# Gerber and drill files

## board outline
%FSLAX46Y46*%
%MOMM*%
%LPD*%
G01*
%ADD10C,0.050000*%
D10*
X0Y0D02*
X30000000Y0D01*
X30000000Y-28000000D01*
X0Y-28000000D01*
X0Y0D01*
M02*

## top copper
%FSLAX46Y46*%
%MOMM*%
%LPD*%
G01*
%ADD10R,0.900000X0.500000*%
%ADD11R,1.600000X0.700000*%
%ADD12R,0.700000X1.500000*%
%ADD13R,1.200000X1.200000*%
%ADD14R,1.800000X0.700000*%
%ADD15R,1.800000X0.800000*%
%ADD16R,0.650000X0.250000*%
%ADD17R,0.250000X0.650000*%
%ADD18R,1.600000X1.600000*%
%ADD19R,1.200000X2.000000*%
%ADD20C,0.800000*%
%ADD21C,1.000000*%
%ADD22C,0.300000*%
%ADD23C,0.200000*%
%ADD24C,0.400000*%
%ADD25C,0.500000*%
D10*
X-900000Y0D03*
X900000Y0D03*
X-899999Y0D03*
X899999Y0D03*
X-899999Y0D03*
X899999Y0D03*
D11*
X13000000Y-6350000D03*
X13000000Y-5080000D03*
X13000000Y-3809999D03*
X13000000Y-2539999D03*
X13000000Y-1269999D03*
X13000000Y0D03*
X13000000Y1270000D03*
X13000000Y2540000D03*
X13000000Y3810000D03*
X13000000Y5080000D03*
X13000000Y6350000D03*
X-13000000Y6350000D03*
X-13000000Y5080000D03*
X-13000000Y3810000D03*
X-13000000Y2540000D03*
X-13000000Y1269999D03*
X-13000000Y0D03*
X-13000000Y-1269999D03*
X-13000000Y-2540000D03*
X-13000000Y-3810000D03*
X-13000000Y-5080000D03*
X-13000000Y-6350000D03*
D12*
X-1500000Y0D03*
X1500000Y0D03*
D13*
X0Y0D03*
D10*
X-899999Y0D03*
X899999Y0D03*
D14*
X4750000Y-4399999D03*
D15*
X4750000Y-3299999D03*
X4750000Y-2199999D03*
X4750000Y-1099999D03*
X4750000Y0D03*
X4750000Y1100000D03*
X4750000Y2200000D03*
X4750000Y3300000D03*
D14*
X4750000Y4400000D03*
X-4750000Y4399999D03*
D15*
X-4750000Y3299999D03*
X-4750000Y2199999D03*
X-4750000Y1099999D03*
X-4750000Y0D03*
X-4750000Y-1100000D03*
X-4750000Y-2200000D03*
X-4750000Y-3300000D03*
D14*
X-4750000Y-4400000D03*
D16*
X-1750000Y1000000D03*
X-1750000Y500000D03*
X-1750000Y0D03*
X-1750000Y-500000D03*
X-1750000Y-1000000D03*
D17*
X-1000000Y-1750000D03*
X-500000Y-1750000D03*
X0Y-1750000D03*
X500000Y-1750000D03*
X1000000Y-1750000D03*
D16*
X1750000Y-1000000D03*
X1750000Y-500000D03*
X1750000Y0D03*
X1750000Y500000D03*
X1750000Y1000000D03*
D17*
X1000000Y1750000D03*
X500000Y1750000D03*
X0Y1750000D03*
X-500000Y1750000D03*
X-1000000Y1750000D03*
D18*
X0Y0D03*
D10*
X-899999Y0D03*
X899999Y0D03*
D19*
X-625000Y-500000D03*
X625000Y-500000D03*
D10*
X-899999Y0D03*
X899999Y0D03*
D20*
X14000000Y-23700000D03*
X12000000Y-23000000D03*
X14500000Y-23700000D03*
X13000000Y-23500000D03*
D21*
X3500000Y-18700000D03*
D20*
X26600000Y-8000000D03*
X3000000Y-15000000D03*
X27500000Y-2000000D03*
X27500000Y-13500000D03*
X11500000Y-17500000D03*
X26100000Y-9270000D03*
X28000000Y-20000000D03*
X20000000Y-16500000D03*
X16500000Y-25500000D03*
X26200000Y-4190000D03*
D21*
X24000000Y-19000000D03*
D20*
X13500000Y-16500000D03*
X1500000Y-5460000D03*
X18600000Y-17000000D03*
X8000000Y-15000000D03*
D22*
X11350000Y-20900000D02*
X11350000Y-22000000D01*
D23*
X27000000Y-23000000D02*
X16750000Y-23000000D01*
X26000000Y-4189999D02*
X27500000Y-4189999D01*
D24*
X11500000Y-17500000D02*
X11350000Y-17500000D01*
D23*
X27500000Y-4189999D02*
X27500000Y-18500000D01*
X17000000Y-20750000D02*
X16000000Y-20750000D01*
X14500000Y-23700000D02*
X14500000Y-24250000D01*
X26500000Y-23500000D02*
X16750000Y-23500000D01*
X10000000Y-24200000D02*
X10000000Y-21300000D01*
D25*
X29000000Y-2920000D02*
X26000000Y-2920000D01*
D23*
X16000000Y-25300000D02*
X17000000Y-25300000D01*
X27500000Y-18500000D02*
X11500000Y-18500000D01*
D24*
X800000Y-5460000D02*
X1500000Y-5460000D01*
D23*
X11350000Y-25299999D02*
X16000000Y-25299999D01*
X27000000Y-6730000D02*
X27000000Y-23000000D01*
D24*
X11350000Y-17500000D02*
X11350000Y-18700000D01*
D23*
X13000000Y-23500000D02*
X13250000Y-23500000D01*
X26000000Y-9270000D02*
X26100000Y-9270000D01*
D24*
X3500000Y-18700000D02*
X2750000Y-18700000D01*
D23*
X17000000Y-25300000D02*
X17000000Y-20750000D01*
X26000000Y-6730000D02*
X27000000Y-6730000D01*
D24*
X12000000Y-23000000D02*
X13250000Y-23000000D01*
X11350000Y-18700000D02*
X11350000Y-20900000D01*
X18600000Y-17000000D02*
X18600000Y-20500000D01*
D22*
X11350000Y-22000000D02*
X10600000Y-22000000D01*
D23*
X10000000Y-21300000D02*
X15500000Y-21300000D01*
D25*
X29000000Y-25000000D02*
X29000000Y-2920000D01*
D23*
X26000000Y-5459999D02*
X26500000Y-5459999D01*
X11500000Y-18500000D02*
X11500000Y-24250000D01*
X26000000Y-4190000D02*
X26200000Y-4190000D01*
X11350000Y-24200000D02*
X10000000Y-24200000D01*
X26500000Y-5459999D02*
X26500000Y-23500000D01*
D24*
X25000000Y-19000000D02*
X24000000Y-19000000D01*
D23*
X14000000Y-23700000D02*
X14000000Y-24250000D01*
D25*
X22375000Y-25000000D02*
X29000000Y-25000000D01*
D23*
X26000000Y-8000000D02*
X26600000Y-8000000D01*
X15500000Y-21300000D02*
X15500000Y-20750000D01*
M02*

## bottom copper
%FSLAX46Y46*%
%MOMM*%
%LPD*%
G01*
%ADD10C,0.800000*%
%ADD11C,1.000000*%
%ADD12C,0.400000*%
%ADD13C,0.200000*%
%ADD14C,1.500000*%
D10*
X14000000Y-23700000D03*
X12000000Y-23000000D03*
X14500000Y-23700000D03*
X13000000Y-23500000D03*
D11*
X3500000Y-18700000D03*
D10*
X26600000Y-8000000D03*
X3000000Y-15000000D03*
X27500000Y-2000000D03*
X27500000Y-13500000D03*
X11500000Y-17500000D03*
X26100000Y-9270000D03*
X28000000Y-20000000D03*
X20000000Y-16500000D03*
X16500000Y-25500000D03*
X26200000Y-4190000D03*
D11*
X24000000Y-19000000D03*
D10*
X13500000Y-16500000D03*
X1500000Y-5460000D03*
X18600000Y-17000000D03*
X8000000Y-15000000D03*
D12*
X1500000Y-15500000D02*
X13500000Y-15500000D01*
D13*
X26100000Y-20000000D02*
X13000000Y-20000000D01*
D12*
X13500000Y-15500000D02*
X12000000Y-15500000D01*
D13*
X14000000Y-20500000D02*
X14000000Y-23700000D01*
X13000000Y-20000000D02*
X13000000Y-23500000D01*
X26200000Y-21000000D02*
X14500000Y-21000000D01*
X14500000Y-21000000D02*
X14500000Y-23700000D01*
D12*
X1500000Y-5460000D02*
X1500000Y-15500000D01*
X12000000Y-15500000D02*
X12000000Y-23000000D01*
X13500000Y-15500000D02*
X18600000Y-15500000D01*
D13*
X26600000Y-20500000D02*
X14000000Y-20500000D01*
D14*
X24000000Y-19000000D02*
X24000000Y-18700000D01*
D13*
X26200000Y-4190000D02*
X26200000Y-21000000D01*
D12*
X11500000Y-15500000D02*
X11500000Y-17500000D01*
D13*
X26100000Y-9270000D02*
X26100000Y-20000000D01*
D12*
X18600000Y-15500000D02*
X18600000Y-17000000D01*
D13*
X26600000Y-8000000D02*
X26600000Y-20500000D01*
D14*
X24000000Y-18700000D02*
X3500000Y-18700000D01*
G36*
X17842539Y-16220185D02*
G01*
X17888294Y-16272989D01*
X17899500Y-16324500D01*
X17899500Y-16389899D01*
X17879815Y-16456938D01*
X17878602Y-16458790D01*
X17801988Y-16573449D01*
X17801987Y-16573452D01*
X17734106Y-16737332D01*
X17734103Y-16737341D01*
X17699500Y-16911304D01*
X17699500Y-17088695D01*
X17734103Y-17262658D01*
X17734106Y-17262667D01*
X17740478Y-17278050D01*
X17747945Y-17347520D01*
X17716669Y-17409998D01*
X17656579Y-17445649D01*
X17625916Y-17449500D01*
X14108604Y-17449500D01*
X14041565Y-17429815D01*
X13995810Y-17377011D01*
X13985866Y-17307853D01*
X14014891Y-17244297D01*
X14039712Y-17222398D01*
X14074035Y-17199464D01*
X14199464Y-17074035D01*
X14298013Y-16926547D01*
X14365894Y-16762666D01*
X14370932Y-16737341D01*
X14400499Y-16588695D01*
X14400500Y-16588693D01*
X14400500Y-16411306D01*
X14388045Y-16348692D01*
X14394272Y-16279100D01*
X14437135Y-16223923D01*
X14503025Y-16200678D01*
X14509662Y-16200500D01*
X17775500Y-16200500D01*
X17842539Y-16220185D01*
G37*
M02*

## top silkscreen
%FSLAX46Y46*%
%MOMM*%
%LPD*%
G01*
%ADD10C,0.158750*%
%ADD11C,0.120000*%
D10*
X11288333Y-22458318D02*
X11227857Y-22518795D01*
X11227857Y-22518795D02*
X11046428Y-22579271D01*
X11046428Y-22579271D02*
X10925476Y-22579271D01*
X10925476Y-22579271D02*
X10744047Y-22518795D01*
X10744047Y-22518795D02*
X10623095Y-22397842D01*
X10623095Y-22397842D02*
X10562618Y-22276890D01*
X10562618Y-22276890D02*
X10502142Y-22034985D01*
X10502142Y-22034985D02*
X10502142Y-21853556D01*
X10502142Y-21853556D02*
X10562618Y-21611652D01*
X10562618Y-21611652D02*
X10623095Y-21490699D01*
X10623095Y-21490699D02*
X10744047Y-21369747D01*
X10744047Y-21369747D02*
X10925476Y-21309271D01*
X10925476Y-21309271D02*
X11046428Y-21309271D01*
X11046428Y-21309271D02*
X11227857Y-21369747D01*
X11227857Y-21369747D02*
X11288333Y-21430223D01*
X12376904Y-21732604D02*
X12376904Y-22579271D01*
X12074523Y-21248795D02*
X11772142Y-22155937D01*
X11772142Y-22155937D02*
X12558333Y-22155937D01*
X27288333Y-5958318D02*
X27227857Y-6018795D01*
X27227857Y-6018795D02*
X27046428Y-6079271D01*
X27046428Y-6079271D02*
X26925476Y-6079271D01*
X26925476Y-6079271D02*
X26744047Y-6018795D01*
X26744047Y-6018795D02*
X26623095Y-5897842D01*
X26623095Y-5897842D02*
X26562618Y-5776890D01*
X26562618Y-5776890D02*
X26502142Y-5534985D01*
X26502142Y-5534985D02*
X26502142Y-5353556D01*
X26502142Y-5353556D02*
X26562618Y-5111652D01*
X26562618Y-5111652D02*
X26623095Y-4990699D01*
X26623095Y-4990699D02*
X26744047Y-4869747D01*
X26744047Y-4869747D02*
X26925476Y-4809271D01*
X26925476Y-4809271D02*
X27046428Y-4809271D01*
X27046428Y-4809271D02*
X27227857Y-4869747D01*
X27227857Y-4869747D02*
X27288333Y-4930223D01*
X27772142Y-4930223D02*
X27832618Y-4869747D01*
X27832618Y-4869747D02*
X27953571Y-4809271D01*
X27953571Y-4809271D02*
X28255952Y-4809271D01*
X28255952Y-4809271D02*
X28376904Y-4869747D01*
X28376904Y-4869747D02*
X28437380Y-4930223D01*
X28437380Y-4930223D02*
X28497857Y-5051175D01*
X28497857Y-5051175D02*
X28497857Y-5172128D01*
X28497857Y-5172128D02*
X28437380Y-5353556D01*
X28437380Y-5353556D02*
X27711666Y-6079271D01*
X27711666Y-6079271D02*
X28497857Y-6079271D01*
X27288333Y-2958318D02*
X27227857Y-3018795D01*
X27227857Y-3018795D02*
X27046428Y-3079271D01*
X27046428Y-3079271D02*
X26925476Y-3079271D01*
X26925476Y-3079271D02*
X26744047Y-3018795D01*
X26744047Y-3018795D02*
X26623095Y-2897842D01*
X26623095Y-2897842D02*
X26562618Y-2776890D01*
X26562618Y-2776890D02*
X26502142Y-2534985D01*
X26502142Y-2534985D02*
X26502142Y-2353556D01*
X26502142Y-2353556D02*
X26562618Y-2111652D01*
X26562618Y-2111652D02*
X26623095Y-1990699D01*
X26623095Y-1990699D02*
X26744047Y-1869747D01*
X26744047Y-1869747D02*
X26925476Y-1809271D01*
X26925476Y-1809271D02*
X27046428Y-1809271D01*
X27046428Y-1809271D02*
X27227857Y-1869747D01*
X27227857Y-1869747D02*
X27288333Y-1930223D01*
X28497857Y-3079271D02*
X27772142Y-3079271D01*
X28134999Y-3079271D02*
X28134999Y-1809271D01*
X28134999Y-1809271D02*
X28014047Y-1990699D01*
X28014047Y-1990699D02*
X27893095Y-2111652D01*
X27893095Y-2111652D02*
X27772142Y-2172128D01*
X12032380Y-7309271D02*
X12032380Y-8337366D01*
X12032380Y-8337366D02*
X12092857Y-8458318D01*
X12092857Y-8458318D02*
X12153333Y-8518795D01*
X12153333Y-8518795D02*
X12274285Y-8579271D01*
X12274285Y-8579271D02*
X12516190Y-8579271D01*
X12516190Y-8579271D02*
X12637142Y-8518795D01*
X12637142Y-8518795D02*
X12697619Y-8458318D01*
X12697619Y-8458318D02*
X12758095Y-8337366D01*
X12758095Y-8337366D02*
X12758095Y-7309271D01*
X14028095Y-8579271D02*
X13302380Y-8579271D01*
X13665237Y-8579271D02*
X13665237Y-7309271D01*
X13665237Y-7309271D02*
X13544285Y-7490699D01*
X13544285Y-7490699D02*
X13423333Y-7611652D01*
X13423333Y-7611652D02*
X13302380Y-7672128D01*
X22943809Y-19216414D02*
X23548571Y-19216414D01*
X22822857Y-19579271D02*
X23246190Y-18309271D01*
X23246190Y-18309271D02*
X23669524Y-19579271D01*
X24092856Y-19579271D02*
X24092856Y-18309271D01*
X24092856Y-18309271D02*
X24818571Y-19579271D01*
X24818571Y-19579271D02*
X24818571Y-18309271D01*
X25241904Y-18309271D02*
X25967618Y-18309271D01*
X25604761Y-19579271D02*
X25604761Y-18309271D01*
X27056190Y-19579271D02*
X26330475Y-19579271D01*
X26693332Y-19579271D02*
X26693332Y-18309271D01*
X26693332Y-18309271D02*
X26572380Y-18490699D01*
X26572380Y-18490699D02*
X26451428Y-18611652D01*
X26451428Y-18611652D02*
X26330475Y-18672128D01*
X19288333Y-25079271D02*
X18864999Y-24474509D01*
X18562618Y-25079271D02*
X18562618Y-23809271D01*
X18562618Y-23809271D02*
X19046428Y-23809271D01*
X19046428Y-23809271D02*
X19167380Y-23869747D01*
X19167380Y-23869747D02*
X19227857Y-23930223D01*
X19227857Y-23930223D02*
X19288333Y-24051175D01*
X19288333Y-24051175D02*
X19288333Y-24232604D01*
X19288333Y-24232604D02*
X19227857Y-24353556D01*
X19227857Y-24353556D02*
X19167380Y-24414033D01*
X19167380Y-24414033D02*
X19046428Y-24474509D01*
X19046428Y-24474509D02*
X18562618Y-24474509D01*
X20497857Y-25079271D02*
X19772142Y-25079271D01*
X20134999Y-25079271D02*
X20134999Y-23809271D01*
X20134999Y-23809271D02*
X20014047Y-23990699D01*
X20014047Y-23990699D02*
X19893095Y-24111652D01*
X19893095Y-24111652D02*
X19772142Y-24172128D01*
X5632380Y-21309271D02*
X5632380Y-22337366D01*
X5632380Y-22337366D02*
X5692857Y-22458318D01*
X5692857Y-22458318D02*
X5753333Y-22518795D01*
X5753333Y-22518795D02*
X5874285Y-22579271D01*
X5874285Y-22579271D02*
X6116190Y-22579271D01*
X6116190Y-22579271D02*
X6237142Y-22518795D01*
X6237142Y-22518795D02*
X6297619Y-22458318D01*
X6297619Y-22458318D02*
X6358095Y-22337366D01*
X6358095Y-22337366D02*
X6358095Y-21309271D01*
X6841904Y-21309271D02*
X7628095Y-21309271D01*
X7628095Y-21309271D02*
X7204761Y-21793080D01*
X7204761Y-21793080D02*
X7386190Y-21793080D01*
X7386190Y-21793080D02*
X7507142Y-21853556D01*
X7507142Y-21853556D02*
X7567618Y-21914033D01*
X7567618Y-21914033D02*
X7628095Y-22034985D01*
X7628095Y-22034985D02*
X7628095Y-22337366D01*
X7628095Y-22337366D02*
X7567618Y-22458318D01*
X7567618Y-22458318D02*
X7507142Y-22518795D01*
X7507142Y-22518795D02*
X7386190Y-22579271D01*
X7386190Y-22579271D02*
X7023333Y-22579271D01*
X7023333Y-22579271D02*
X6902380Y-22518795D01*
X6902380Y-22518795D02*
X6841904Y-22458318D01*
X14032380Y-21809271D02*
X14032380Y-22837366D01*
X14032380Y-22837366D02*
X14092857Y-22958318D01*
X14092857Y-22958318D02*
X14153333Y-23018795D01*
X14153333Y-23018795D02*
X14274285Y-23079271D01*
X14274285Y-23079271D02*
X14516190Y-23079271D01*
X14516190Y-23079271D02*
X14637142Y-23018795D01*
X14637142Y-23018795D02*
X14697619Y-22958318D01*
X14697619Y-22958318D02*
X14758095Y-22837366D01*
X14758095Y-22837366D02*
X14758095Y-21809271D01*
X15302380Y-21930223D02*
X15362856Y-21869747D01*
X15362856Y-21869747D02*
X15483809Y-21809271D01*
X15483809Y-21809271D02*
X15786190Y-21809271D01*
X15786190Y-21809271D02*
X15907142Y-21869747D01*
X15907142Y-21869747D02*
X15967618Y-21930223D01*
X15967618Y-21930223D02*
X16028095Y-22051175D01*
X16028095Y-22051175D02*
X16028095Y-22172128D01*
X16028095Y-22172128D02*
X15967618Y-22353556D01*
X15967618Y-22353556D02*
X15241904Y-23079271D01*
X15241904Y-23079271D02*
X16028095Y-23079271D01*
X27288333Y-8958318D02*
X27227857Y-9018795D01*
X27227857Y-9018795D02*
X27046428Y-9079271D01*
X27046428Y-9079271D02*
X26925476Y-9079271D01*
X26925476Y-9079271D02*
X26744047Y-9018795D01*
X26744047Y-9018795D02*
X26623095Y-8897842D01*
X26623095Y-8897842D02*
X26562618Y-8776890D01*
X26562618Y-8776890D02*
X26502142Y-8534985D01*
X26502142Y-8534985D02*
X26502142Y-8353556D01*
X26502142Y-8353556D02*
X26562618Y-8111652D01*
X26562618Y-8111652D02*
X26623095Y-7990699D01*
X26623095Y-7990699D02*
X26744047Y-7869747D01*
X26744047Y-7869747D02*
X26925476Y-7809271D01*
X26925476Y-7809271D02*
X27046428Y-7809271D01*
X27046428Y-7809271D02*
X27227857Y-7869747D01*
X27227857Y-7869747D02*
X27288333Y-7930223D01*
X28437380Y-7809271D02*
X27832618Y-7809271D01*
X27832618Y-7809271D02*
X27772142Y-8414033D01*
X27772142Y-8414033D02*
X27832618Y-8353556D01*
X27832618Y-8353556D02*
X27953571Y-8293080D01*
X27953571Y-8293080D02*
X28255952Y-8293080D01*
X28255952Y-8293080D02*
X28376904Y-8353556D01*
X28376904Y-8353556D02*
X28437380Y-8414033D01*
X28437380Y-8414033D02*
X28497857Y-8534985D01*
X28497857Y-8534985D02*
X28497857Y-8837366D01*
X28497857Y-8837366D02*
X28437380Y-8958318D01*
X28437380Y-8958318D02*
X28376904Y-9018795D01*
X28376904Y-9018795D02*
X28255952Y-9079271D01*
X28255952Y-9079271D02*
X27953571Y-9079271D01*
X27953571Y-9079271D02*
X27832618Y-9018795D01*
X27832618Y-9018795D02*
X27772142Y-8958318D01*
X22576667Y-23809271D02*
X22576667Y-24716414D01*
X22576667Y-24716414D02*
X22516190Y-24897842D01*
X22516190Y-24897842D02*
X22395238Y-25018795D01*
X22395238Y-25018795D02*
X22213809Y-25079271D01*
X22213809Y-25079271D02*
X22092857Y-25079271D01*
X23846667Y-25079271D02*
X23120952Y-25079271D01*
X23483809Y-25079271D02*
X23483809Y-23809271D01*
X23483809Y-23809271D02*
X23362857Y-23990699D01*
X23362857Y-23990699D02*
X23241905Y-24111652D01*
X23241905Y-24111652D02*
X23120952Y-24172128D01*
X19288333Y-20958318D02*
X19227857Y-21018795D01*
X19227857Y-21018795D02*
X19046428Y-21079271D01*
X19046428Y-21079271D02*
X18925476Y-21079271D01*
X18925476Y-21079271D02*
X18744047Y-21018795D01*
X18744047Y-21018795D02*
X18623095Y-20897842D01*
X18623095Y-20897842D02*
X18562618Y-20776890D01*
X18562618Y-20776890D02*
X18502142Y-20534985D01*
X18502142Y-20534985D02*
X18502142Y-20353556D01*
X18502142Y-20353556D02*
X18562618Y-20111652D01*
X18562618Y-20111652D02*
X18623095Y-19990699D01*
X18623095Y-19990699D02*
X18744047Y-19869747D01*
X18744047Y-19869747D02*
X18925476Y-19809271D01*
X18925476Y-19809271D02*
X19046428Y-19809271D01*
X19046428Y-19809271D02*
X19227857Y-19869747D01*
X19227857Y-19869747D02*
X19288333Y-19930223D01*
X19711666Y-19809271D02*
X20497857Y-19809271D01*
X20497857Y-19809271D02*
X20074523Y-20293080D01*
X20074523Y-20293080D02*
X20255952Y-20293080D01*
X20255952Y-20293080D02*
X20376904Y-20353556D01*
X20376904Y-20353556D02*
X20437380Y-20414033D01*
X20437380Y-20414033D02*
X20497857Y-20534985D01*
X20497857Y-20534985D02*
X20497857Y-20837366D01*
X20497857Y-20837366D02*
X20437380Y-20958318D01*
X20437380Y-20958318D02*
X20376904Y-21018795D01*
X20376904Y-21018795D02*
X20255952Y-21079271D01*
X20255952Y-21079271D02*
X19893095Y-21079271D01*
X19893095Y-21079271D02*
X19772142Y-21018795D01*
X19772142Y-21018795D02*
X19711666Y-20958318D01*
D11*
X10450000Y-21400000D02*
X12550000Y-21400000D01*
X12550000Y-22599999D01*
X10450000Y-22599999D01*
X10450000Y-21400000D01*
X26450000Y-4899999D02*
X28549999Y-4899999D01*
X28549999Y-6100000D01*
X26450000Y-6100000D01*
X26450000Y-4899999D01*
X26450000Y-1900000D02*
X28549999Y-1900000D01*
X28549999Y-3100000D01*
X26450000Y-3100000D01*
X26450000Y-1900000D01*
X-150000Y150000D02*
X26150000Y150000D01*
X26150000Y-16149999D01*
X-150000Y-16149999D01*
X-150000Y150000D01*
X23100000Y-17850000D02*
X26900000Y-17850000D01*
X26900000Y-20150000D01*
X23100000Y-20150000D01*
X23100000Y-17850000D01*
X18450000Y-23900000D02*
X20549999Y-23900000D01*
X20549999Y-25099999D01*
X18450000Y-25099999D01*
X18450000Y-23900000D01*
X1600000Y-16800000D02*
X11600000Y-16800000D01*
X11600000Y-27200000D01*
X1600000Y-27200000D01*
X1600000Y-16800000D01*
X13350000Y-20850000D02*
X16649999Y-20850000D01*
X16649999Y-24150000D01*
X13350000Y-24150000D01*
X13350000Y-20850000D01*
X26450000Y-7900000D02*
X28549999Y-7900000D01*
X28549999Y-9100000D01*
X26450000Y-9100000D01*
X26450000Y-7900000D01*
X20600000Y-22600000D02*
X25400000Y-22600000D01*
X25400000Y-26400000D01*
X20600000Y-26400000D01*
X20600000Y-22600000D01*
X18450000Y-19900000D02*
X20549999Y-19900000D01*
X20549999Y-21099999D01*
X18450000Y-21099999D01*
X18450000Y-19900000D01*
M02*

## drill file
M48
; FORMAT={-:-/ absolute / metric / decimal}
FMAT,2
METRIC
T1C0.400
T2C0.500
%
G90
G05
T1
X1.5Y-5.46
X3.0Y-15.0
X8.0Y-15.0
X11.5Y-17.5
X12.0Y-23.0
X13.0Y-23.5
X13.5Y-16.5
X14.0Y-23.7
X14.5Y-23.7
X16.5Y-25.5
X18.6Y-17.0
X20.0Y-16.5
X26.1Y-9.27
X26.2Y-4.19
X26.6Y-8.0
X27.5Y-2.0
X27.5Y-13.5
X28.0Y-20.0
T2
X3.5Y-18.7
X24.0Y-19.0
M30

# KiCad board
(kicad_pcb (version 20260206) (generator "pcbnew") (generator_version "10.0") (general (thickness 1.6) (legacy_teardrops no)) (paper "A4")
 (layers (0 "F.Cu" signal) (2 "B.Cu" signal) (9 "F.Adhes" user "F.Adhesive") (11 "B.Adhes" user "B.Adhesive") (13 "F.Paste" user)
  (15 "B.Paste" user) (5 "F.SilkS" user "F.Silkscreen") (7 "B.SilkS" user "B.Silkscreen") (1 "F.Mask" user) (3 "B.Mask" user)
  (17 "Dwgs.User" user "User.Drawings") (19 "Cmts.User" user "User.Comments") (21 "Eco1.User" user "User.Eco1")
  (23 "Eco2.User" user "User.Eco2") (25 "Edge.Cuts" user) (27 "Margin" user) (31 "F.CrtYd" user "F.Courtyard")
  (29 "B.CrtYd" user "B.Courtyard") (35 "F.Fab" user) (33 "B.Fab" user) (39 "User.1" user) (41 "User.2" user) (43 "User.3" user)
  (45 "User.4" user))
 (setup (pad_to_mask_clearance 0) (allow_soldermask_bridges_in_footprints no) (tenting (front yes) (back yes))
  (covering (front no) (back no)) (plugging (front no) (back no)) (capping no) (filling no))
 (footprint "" (layer "F.Cu") (at 11.5 22)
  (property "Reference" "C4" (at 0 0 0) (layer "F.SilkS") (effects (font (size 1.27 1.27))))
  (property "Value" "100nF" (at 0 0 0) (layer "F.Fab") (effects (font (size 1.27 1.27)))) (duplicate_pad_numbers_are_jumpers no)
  (fp_rect (start -1.05 -0.6) (end 1.05 0.599999) (stroke (width 0.12) (type default)) (fill no) (layer "F.SilkS"))
  (pad "1" smd rect (at -12.4 -22) (size 0.9 0.5) (layers "F.Cu" "F.Mask" "F.Paste") (thermal_bridge_angle 45))
  (pad "2" smd rect (at -10.6 -22) (size 0.9 0.5) (layers "F.Cu" "F.Mask" "F.Paste") (thermal_bridge_angle 45)))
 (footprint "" (layer "F.Cu") (at 27.5 5.5)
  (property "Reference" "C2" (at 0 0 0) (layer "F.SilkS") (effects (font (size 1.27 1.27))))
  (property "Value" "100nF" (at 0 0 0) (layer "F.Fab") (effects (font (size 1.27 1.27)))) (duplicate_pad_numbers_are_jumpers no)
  (fp_rect (start -1.05 -0.600001) (end 1.049999 0.6) (stroke (width 0.12) (type default)) (fill no) (layer "F.SilkS"))
  (pad "1" smd rect (at -28.399999 -5.5) (size 0.9 0.5) (layers "F.Cu" "F.Mask" "F.Paste") (thermal_bridge_angle 45))
  (pad "2" smd rect (at -26.600001 -5.5) (size 0.9 0.5) (layers "F.Cu" "F.Mask" "F.Paste") (thermal_bridge_angle 45)))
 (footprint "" (layer "F.Cu") (at 27.5 2.5)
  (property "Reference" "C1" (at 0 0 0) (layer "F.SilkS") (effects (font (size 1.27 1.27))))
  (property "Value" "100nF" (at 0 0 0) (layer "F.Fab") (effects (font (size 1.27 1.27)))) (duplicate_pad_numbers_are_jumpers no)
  (fp_rect (start -1.05 -0.6) (end 1.049999 0.6) (stroke (width 0.12) (type default)) (fill no) (layer "F.SilkS"))
  (pad "1" smd rect (at -28.399999 -2.5) (size 0.9 0.5) (layers "F.Cu" "F.Mask" "F.Paste") (thermal_bridge_angle 45))
  (pad "2" smd rect (at -26.600001 -2.5) (size 0.9 0.5) (layers "F.Cu" "F.Mask" "F.Paste") (thermal_bridge_angle 45)))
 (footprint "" (layer "F.Cu") (at 13 8)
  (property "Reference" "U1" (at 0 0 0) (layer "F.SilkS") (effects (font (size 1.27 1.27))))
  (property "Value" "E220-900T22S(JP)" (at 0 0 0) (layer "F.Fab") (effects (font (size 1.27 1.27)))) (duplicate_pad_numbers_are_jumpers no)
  (fp_rect (start -13.15 -8.15) (end 13.15 8.149999) (stroke (width 0.12) (type default)) (fill no) (layer "F.SilkS"))
  (pad "1" smd rect (at 0 -1.65) (size 1.6 0.7) (layers "F.Cu" "F.Mask" "F.Paste") (thermal_bridge_angle 45))
  (pad "2" smd rect (at 0 -2.92) (size 1.6 0.7) (layers "F.Cu" "F.Mask" "F.Paste") (thermal_bridge_angle 45))
  (pad "3" smd rect (at 0 -4.190001) (size 1.6 0.7) (layers "F.Cu" "F.Mask" "F.Paste") (thermal_bridge_angle 45))
  (pad "4" smd rect (at 0 -5.460001) (size 1.6 0.7) (layers "F.Cu" "F.Mask" "F.Paste") (thermal_bridge_angle 45))
  (pad "5" smd rect (at 0 -6.730001) (size 1.6 0.7) (layers "F.Cu" "F.Mask" "F.Paste") (thermal_bridge_angle 45))
  (pad "6" smd rect (at 0 -8) (size 1.6 0.7) (layers "F.Cu" "F.Mask" "F.Paste") (thermal_bridge_angle 45))
  (pad "7" smd rect (at 0 -9.27) (size 1.6 0.7) (layers "F.Cu" "F.Mask" "F.Paste") (thermal_bridge_angle 45))
  (pad "8" smd rect (at 0 -10.54) (size 1.6 0.7) (layers "F.Cu" "F.Mask" "F.Paste") (thermal_bridge_angle 45))
  (pad "9" smd rect (at 0 -11.81) (size 1.6 0.7) (layers "F.Cu" "F.Mask" "F.Paste") (thermal_bridge_angle 45))
  (pad "10" smd rect (at 0 -13.08) (size 1.6 0.7) (layers "F.Cu" "F.Mask" "F.Paste") (thermal_bridge_angle 45))
  (pad "11" smd rect (at 0 -14.35) (size 1.6 0.7) (layers "F.Cu" "F.Mask" "F.Paste") (thermal_bridge_angle 45))
  (pad "12" smd rect (at -26 -14.35) (size 1.6 0.7) (layers "F.Cu" "F.Mask" "F.Paste") (thermal_bridge_angle 45))
  (pad "13" smd rect (at -26 -13.08) (size 1.6 0.7) (layers "F.Cu" "F.Mask" "F.Paste") (thermal_bridge_angle 45))
  (pad "14" smd rect (at -26 -11.81) (size 1.6 0.7) (layers "F.Cu" "F.Mask" "F.Paste") (thermal_bridge_angle 45))
  (pad "15" smd rect (at -26 -10.54) (size 1.6 0.7) (layers "F.Cu" "F.Mask" "F.Paste") (thermal_bridge_angle 45))
  (pad "16" smd rect (at -26 -9.269999) (size 1.6 0.7) (layers "F.Cu" "F.Mask" "F.Paste") (thermal_bridge_angle 45))
  (pad "17" smd rect (at -26 -8) (size 1.6 0.7) (layers "F.Cu" "F.Mask" "F.Paste") (thermal_bridge_angle 45))
  (pad "18" smd rect (at -26 -6.730001) (size 1.6 0.7) (layers "F.Cu" "F.Mask" "F.Paste") (thermal_bridge_angle 45))
  (pad "19" smd rect (at -26 -5.46) (size 1.6 0.7) (layers "F.Cu" "F.Mask" "F.Paste") (thermal_bridge_angle 45))
  (pad "20" smd rect (at -26 -4.19) (size 1.6 0.7) (layers "F.Cu" "F.Mask" "F.Paste") (thermal_bridge_angle 45))
  (pad "21" smd rect (at -26 -2.92) (size 1.6 0.7) (layers "F.Cu" "F.Mask" "F.Paste") (thermal_bridge_angle 45))
  (pad "22" smd rect (at -26 -1.65) (size 1.6 0.7) (layers "F.Cu" "F.Mask" "F.Paste") (thermal_bridge_angle 45)))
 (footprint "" (layer "F.Cu") (at 25 19)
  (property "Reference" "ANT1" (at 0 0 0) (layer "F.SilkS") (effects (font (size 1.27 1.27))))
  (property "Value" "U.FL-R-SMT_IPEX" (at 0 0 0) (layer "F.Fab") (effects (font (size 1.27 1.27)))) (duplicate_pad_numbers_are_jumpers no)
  (fp_rect (start -1.9 -1.15) (end 1.9 1.15) (stroke (width 0.12) (type default)) (fill no) (layer "F.SilkS"))
  (pad "G1" smd rect (at -26.5 -19) (size 0.7 1.5) (layers "F.Cu" "F.Mask" "F.Paste") (thermal_bridge_angle 45))
  (pad "G2" smd rect (at -23.5 -19) (size 0.7 1.5) (layers "F.Cu" "F.Mask" "F.Paste") (thermal_bridge_angle 45))
  (pad "S" smd rect (at -25 -19) (size 1.2 1.2) (layers "F.Cu" "F.Mask" "F.Paste") (thermal_bridge_angle 45)))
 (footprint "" (layer "F.Cu") (at 19.5 24.5)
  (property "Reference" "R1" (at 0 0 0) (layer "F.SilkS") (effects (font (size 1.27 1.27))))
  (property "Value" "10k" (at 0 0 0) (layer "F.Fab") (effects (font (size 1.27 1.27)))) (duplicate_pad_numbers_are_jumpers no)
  (fp_rect (start -1.05 -0.6) (end 1.049999 0.599999) (stroke (width 0.12) (type default)) (fill no) (layer "F.SilkS"))
  (pad "1" smd rect (at -20.399999 -24.5) (size 0.9 0.5) (layers "F.Cu" "F.Mask" "F.Paste") (thermal_bridge_angle 45))
  (pad "2" smd rect (at -18.600001 -24.5) (size 0.9 0.5) (layers "F.Cu" "F.Mask" "F.Paste") (thermal_bridge_angle 45)))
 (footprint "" (layer "F.Cu") (at 6.6 22)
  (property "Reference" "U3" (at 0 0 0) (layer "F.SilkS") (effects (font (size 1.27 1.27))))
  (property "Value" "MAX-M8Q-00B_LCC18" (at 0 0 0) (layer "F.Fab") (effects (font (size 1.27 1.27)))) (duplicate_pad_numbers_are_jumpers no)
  (fp_rect (start -5 -5.2) (end 5 5.2) (stroke (width 0.12) (type default)) (fill no) (layer "F.SilkS"))
  (pad "1" smd rect (at -1.85 -17.600001) (size 1.8 0.7) (layers "F.Cu" "F.Mask" "F.Paste") (thermal_bridge_angle 45))
  (pad "2" smd rect (at -1.85 -18.700001) (size 1.8 0.8) (layers "F.Cu" "F.Mask" "F.Paste") (thermal_bridge_angle 45))
  (pad "3" smd rect (at -1.85 -19.800001) (size 1.8 0.8) (layers "F.Cu" "F.Mask" "F.Paste") (thermal_bridge_angle 45))
  (pad "4" smd rect (at -1.85 -20.900001) (size 1.8 0.8) (layers "F.Cu" "F.Mask" "F.Paste") (thermal_bridge_angle 45))
  (pad "5" smd rect (at -1.85 -22) (size 1.8 0.8) (layers "F.Cu" "F.Mask" "F.Paste") (thermal_bridge_angle 45))
  (pad "6" smd rect (at -1.85 -23.1) (size 1.8 0.8) (layers "F.Cu" "F.Mask" "F.Paste") (thermal_bridge_angle 45))
  (pad "7" smd rect (at -1.85 -24.2) (size 1.8 0.8) (layers "F.Cu" "F.Mask" "F.Paste") (thermal_bridge_angle 45))
  (pad "8" smd rect (at -1.85 -25.3) (size 1.8 0.8) (layers "F.Cu" "F.Mask" "F.Paste") (thermal_bridge_angle 45))
  (pad "9" smd rect (at -1.85 -26.4) (size 1.8 0.7) (layers "F.Cu" "F.Mask" "F.Paste") (thermal_bridge_angle 45))
  (pad "10" smd rect (at -11.35 -26.399999) (size 1.8 0.7) (layers "F.Cu" "F.Mask" "F.Paste") (thermal_bridge_angle 45))
  (pad "11" smd rect (at -11.35 -25.299999) (size 1.8 0.8) (layers "F.Cu" "F.Mask" "F.Paste") (thermal_bridge_angle 45))
  (pad "12" smd rect (at -11.35 -24.199999) (size 1.8 0.8) (layers "F.Cu" "F.Mask" "F.Paste") (thermal_bridge_angle 45))
  (pad "13" smd rect (at -11.35 -23.099999) (size 1.8 0.8) (layers "F.Cu" "F.Mask" "F.Paste") (thermal_bridge_angle 45))
  (pad "14" smd rect (at -11.35 -22) (size 1.8 0.8) (layers "F.Cu" "F.Mask" "F.Paste") (thermal_bridge_angle 45))
  (pad "15" smd rect (at -11.35 -20.9) (size 1.8 0.8) (layers "F.Cu" "F.Mask" "F.Paste") (thermal_bridge_angle 45))
  (pad "16" smd rect (at -11.35 -19.8) (size 1.8 0.8) (layers "F.Cu" "F.Mask" "F.Paste") (thermal_bridge_angle 45))
  (pad "17" smd rect (at -11.35 -18.7) (size 1.8 0.8) (layers "F.Cu" "F.Mask" "F.Paste") (thermal_bridge_angle 45))
  (pad "18" smd rect (at -11.35 -17.6) (size 1.8 0.7) (layers "F.Cu" "F.Mask" "F.Paste") (thermal_bridge_angle 45)))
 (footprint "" (layer "F.Cu") (at 15 22.5)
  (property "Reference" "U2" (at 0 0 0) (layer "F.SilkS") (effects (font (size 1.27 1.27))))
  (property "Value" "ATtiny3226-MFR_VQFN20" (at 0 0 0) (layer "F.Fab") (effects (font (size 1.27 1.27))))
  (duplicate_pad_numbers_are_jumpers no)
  (fp_rect (start -1.65 -1.65) (end 1.649999 1.65) (stroke (width 0.12) (type default)) (fill no) (layer "F.SilkS"))
  (pad "1" smd rect (at -16.75 -23.5) (size 0.65 0.25) (layers "F.Cu" "F.Mask" "F.Paste") (thermal_bridge_angle 45))
  (pad "2" smd rect (at -16.75 -23) (size 0.65 0.25) (layers "F.Cu" "F.Mask" "F.Paste") (thermal_bridge_angle 45))
  (pad "3" smd rect (at -16.75 -22.5) (size 0.65 0.25) (layers "F.Cu" "F.Mask" "F.Paste") (thermal_bridge_angle 45))
  (pad "4" smd rect (at -16.75 -22) (size 0.65 0.25) (layers "F.Cu" "F.Mask" "F.Paste") (thermal_bridge_angle 45))
  (pad "5" smd rect (at -16.75 -21.5) (size 0.65 0.25) (layers "F.Cu" "F.Mask" "F.Paste") (thermal_bridge_angle 45))
  (pad "6" smd rect (at -16 -20.75) (size 0.25 0.65) (layers "F.Cu" "F.Mask" "F.Paste") (thermal_bridge_angle 45))
  (pad "7" smd rect (at -15.5 -20.75) (size 0.25 0.65) (layers "F.Cu" "F.Mask" "F.Paste") (thermal_bridge_angle 45))
  (pad "8" smd rect (at -15 -20.75) (size 0.25 0.65) (layers "F.Cu" "F.Mask" "F.Paste") (thermal_bridge_angle 45))
  (pad "9" smd rect (at -14.5 -20.75) (size 0.25 0.65) (layers "F.Cu" "F.Mask" "F.Paste") (thermal_bridge_angle 45))
  (pad "10" smd rect (at -14 -20.75) (size 0.25 0.65) (layers "F.Cu" "F.Mask" "F.Paste") (thermal_bridge_angle 45))
  (pad "11" smd rect (at -13.25 -21.5) (size 0.65 0.25) (layers "F.Cu" "F.Mask" "F.Paste") (thermal_bridge_angle 45))
  (pad "12" smd rect (at -13.25 -22) (size 0.65 0.25) (layers "F.Cu" "F.Mask" "F.Paste") (thermal_bridge_angle 45))
  (pad "13" smd rect (at -13.25 -22.5) (size 0.65 0.25) (layers "F.Cu" "F.Mask" "F.Paste") (thermal_bridge_angle 45))
  (pad "14" smd rect (at -13.25 -23) (size 0.65 0.25) (layers "F.Cu" "F.Mask" "F.Paste") (thermal_bridge_angle 45))
  (pad "15" smd rect (at -13.25 -23.5) (size 0.65 0.25) (layers "F.Cu" "F.Mask" "F.Paste") (thermal_bridge_angle 45))
  (pad "16" smd rect (at -14 -24.25) (size 0.25 0.65) (layers "F.Cu" "F.Mask" "F.Paste") (thermal_bridge_angle 45))
  (pad "17" smd rect (at -14.5 -24.25) (size 0.25 0.65) (layers "F.Cu" "F.Mask" "F.Paste") (thermal_bridge_angle 45))
  (pad "18" smd rect (at -15 -24.25) (size 0.25 0.65) (layers "F.Cu" "F.Mask" "F.Paste") (thermal_bridge_angle 45))
  (pad "19" smd rect (at -15.5 -24.25) (size 0.25 0.65) (layers "F.Cu" "F.Mask" "F.Paste") (thermal_bridge_angle 45))
  (pad "20" smd rect (at -16 -24.25) (size 0.25 0.65) (layers "F.Cu" "F.Mask" "F.Paste") (thermal_bridge_angle 45))
  (pad "EP" smd rect (at -15 -22.5) (size 1.6 1.6) (layers "F.Cu" "F.Mask" "F.Paste") (thermal_bridge_angle 45)))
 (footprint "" (layer "F.Cu") (at 27.5 8.5)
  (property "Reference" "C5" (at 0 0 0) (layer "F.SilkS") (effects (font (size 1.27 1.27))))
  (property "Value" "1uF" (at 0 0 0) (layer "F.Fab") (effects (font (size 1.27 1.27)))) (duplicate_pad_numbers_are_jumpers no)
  (fp_rect (start -1.05 -0.6) (end 1.049999 0.6) (stroke (width 0.12) (type default)) (fill no) (layer "F.SilkS"))
  (pad "1" smd rect (at -28.399999 -8.5) (size 0.9 0.5) (layers "F.Cu" "F.Mask" "F.Paste") (thermal_bridge_angle 45))
  (pad "2" smd rect (at -26.600001 -8.5) (size 0.9 0.5) (layers "F.Cu" "F.Mask" "F.Paste") (thermal_bridge_angle 45)))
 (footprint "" (layer "F.Cu") (at 23 24.5)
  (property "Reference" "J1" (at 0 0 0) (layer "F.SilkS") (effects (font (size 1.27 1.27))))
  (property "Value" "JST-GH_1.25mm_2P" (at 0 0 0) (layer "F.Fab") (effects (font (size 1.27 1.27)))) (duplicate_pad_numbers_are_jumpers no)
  (fp_rect (start -2.4 -1.9) (end 2.4 1.9) (stroke (width 0.12) (type default)) (fill no) (layer "F.SilkS"))
  (pad "1" smd rect (at -23.625 -24) (size 1.2 2) (layers "F.Cu" "F.Mask" "F.Paste") (thermal_bridge_angle 45))
  (pad "2" smd rect (at -22.375 -24) (size 1.2 2) (layers "F.Cu" "F.Mask" "F.Paste") (thermal_bridge_angle 45)))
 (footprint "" (layer "F.Cu") (at 19.5 20.5)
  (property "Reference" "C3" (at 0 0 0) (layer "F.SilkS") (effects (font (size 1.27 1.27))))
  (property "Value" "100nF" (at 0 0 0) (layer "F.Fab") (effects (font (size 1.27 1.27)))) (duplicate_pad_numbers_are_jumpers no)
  (fp_rect (start -1.05 -0.6) (end 1.049999 0.599999) (stroke (width 0.12) (type default)) (fill no) (layer "F.SilkS"))
  (pad "1" smd rect (at -20.399999 -20.5) (size 0.9 0.5) (layers "F.Cu" "F.Mask" "F.Paste") (thermal_bridge_angle 45))
  (pad "2" smd rect (at -18.600001 -20.5) (size 0.9 0.5) (layers "F.Cu" "F.Mask" "F.Paste") (thermal_bridge_angle 45)))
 (gr_rect (start 0 0) (end 30 28) (stroke (width 0.05) (type default)) (fill no) (layer "Edge.Cuts"))
 (segment (start 11.35 20.9) (end 11.35 22) (width 0.3) (layer "F.Cu") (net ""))
 (segment (start 27 23) (end 16.75 23) (width 0.2) (layer "F.Cu") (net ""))
 (segment (start 26 4.189999) (end 27.5 4.189999) (width 0.2) (layer "F.Cu") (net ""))
 (segment (start 11.5 17.5) (end 11.35 17.5) (width 0.4) (layer "F.Cu") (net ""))
 (segment (start 27.5 4.189999) (end 27.5 18.5) (width 0.2) (layer "F.Cu") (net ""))
 (segment (start 17 20.75) (end 16 20.75) (width 0.2) (layer "F.Cu") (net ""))
 (segment (start 14.5 23.7) (end 14.5 24.25) (width 0.2) (layer "F.Cu") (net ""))
 (segment (start 26.5 23.5) (end 16.75 23.5) (width 0.2) (layer "F.Cu") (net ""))
 (segment (start 10 24.2) (end 10 21.3) (width 0.2) (layer "F.Cu") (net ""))
 (segment (start 29 2.92) (end 26 2.92) (width 0.5) (layer "F.Cu") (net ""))
 (segment (start 16 25.3) (end 17 25.3) (width 0.2) (layer "F.Cu") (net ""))
 (segment (start 27.5 18.5) (end 11.5 18.5) (width 0.2) (layer "F.Cu") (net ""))
 (segment (start 0.8 5.46) (end 1.5 5.46) (width 0.4) (layer "F.Cu") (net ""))
 (segment (start 11.35 25.299999) (end 16 25.299999) (width 0.2) (layer "F.Cu") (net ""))
 (segment (start 27 6.73) (end 27 23) (width 0.2) (layer "F.Cu") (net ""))
 (segment (start 11.35 17.5) (end 11.35 18.7) (width 0.4) (layer "F.Cu") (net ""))
 (segment (start 13 23.5) (end 13.25 23.5) (width 0.2) (layer "F.Cu") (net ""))
 (segment (start 26 9.27) (end 26.1 9.27) (width 0.2) (layer "F.Cu") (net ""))
 (segment (start 3.5 18.7) (end 2.75 18.7) (width 0.4) (layer "F.Cu") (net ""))
 (segment (start 17 25.3) (end 17 20.75) (width 0.2) (layer "F.Cu") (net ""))
 (segment (start 26 6.73) (end 27 6.73) (width 0.2) (layer "F.Cu") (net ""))
 (segment (start 12 23) (end 13.25 23) (width 0.4) (layer "F.Cu") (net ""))
 (segment (start 11.35 18.7) (end 11.35 20.9) (width 0.4) (layer "F.Cu") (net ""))
 (segment (start 18.6 17) (end 18.6 20.5) (width 0.4) (layer "F.Cu") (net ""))
 (segment (start 11.35 22) (end 10.6 22) (width 0.3) (layer "F.Cu") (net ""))
 (segment (start 10 21.3) (end 15.5 21.3) (width 0.2) (layer "F.Cu") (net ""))
 (segment (start 29 25) (end 29 2.92) (width 0.5) (layer "F.Cu") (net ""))
 (segment (start 26 5.459999) (end 26.5 5.459999) (width 0.2) (layer "F.Cu") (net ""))
 (segment (start 11.5 18.5) (end 11.5 24.25) (width 0.2) (layer "F.Cu") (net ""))
 (segment (start 26 4.19) (end 26.2 4.19) (width 0.2) (layer "F.Cu") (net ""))
 (segment (start 11.35 24.2) (end 10 24.2) (width 0.2) (layer "F.Cu") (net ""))
 (segment (start 26.5 5.459999) (end 26.5 23.5) (width 0.2) (layer "F.Cu") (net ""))
 (segment (start 25 19) (end 24 19) (width 0.4) (layer "F.Cu") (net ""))
 (segment (start 14 23.7) (end 14 24.25) (width 0.2) (layer "F.Cu") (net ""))
 (segment (start 22.375 25) (end 29 25) (width 0.5) (layer "F.Cu") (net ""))
 (segment (start 26 8) (end 26.6 8) (width 0.2) (layer "F.Cu") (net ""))
 (segment (start 15.5 21.3) (end 15.5 20.75) (width 0.2) (layer "F.Cu") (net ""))
 (via (at 14 23.7) (size 0.8) (drill 0.4) (layers "F.Cu" "B.Cu") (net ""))
 (via (at 12 23) (size 0.8) (drill 0.4) (layers "F.Cu" "B.Cu") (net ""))
 (via (at 14.5 23.7) (size 0.8) (drill 0.4) (layers "F.Cu" "B.Cu") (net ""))
 (via (at 13 23.5) (size 0.8) (drill 0.4) (layers "F.Cu" "B.Cu") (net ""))
 (via (at 3.5 18.7) (size 1) (drill 0.5) (layers "F.Cu" "B.Cu") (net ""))
 (via (at 26.6 8) (size 0.8) (drill 0.4) (layers "F.Cu" "B.Cu") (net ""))
 (via (at 3 15) (size 0.8) (drill 0.4) (layers "F.Cu" "B.Cu") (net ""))
 (via (at 27.5 2) (size 0.8) (drill 0.4) (layers "F.Cu" "B.Cu") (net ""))
 (via (at 27.5 13.5) (size 0.8) (drill 0.4) (layers "F.Cu" "B.Cu") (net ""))
 (via (at 11.5 17.5) (size 0.8) (drill 0.4) (layers "F.Cu" "B.Cu") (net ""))
 (via (at 26.1 9.27) (size 0.8) (drill 0.4) (layers "F.Cu" "B.Cu") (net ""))
 (via (at 28 20) (size 0.8) (drill 0.4) (layers "F.Cu" "B.Cu") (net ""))
 (via (at 20 16.5) (size 0.8) (drill 0.4) (layers "F.Cu" "B.Cu") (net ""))
 (via (at 16.5 25.5) (size 0.8) (drill 0.4) (layers "F.Cu" "B.Cu") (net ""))
 (via (at 26.2 4.19) (size 0.8) (drill 0.4) (layers "F.Cu" "B.Cu") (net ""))
 (via (at 24 19) (size 1) (drill 0.5) (layers "F.Cu" "B.Cu") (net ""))
 (via (at 13.5 16.5) (size 0.8) (drill 0.4) (layers "F.Cu" "B.Cu") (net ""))
 (via (at 1.5 5.46) (size 0.8) (drill 0.4) (layers "F.Cu" "B.Cu") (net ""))
 (via (at 18.6 17) (size 0.8) (drill 0.4) (layers "F.Cu" "B.Cu") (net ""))
 (via (at 8 15) (size 0.8) (drill 0.4) (layers "F.Cu" "B.Cu") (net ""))
 (segment (start 1.5 15.5) (end 13.5 15.5) (width 0.4) (layer "B.Cu") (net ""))
 (segment (start 26.1 20) (end 13 20) (width 0.2) (layer "B.Cu") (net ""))
 (segment (start 13.5 15.5) (end 12 15.5) (width 0.4) (layer "B.Cu") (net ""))
 (segment (start 14 20.5) (end 14 23.7) (width 0.2) (layer "B.Cu") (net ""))
 (segment (start 13 20) (end 13 23.5) (width 0.2) (layer "B.Cu") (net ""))
 (segment (start 26.2 21) (end 14.5 21) (width 0.2) (layer "B.Cu") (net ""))
 (segment (start 14.5 21) (end 14.5 23.7) (width 0.2) (layer "B.Cu") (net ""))
 (segment (start 1.5 5.46) (end 1.5 15.5) (width 0.4) (layer "B.Cu") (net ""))
 (segment (start 12 15.5) (end 12 23) (width 0.4) (layer "B.Cu") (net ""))
 (segment (start 13.5 15.5) (end 18.6 15.5) (width 0.4) (layer "B.Cu") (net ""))
 (segment (start 26.6 20.5) (end 14 20.5) (width 0.2) (layer "B.Cu") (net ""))
 (segment (start 24 19) (end 24 18.7) (width 1.5) (layer "B.Cu") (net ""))
 (segment (start 26.2 4.19) (end 26.2 21) (width 0.2) (layer "B.Cu") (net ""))
 (segment (start 11.5 15.5) (end 11.5 17.5) (width 0.4) (layer "B.Cu") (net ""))
 (segment (start 26.1 9.27) (end 26.1 20) (width 0.2) (layer "B.Cu") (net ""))
 (segment (start 18.6 15.5) (end 18.6 17) (width 0.4) (layer "B.Cu") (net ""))
 (segment (start 26.6 8) (end 26.6 20.5) (width 0.2) (layer "B.Cu") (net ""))
 (segment (start 24 18.7) (end 3.5 18.7) (width 1.5) (layer "B.Cu") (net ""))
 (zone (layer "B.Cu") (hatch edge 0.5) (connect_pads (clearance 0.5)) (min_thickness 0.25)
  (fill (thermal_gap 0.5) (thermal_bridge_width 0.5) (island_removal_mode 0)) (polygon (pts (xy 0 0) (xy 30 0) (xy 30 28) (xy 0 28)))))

